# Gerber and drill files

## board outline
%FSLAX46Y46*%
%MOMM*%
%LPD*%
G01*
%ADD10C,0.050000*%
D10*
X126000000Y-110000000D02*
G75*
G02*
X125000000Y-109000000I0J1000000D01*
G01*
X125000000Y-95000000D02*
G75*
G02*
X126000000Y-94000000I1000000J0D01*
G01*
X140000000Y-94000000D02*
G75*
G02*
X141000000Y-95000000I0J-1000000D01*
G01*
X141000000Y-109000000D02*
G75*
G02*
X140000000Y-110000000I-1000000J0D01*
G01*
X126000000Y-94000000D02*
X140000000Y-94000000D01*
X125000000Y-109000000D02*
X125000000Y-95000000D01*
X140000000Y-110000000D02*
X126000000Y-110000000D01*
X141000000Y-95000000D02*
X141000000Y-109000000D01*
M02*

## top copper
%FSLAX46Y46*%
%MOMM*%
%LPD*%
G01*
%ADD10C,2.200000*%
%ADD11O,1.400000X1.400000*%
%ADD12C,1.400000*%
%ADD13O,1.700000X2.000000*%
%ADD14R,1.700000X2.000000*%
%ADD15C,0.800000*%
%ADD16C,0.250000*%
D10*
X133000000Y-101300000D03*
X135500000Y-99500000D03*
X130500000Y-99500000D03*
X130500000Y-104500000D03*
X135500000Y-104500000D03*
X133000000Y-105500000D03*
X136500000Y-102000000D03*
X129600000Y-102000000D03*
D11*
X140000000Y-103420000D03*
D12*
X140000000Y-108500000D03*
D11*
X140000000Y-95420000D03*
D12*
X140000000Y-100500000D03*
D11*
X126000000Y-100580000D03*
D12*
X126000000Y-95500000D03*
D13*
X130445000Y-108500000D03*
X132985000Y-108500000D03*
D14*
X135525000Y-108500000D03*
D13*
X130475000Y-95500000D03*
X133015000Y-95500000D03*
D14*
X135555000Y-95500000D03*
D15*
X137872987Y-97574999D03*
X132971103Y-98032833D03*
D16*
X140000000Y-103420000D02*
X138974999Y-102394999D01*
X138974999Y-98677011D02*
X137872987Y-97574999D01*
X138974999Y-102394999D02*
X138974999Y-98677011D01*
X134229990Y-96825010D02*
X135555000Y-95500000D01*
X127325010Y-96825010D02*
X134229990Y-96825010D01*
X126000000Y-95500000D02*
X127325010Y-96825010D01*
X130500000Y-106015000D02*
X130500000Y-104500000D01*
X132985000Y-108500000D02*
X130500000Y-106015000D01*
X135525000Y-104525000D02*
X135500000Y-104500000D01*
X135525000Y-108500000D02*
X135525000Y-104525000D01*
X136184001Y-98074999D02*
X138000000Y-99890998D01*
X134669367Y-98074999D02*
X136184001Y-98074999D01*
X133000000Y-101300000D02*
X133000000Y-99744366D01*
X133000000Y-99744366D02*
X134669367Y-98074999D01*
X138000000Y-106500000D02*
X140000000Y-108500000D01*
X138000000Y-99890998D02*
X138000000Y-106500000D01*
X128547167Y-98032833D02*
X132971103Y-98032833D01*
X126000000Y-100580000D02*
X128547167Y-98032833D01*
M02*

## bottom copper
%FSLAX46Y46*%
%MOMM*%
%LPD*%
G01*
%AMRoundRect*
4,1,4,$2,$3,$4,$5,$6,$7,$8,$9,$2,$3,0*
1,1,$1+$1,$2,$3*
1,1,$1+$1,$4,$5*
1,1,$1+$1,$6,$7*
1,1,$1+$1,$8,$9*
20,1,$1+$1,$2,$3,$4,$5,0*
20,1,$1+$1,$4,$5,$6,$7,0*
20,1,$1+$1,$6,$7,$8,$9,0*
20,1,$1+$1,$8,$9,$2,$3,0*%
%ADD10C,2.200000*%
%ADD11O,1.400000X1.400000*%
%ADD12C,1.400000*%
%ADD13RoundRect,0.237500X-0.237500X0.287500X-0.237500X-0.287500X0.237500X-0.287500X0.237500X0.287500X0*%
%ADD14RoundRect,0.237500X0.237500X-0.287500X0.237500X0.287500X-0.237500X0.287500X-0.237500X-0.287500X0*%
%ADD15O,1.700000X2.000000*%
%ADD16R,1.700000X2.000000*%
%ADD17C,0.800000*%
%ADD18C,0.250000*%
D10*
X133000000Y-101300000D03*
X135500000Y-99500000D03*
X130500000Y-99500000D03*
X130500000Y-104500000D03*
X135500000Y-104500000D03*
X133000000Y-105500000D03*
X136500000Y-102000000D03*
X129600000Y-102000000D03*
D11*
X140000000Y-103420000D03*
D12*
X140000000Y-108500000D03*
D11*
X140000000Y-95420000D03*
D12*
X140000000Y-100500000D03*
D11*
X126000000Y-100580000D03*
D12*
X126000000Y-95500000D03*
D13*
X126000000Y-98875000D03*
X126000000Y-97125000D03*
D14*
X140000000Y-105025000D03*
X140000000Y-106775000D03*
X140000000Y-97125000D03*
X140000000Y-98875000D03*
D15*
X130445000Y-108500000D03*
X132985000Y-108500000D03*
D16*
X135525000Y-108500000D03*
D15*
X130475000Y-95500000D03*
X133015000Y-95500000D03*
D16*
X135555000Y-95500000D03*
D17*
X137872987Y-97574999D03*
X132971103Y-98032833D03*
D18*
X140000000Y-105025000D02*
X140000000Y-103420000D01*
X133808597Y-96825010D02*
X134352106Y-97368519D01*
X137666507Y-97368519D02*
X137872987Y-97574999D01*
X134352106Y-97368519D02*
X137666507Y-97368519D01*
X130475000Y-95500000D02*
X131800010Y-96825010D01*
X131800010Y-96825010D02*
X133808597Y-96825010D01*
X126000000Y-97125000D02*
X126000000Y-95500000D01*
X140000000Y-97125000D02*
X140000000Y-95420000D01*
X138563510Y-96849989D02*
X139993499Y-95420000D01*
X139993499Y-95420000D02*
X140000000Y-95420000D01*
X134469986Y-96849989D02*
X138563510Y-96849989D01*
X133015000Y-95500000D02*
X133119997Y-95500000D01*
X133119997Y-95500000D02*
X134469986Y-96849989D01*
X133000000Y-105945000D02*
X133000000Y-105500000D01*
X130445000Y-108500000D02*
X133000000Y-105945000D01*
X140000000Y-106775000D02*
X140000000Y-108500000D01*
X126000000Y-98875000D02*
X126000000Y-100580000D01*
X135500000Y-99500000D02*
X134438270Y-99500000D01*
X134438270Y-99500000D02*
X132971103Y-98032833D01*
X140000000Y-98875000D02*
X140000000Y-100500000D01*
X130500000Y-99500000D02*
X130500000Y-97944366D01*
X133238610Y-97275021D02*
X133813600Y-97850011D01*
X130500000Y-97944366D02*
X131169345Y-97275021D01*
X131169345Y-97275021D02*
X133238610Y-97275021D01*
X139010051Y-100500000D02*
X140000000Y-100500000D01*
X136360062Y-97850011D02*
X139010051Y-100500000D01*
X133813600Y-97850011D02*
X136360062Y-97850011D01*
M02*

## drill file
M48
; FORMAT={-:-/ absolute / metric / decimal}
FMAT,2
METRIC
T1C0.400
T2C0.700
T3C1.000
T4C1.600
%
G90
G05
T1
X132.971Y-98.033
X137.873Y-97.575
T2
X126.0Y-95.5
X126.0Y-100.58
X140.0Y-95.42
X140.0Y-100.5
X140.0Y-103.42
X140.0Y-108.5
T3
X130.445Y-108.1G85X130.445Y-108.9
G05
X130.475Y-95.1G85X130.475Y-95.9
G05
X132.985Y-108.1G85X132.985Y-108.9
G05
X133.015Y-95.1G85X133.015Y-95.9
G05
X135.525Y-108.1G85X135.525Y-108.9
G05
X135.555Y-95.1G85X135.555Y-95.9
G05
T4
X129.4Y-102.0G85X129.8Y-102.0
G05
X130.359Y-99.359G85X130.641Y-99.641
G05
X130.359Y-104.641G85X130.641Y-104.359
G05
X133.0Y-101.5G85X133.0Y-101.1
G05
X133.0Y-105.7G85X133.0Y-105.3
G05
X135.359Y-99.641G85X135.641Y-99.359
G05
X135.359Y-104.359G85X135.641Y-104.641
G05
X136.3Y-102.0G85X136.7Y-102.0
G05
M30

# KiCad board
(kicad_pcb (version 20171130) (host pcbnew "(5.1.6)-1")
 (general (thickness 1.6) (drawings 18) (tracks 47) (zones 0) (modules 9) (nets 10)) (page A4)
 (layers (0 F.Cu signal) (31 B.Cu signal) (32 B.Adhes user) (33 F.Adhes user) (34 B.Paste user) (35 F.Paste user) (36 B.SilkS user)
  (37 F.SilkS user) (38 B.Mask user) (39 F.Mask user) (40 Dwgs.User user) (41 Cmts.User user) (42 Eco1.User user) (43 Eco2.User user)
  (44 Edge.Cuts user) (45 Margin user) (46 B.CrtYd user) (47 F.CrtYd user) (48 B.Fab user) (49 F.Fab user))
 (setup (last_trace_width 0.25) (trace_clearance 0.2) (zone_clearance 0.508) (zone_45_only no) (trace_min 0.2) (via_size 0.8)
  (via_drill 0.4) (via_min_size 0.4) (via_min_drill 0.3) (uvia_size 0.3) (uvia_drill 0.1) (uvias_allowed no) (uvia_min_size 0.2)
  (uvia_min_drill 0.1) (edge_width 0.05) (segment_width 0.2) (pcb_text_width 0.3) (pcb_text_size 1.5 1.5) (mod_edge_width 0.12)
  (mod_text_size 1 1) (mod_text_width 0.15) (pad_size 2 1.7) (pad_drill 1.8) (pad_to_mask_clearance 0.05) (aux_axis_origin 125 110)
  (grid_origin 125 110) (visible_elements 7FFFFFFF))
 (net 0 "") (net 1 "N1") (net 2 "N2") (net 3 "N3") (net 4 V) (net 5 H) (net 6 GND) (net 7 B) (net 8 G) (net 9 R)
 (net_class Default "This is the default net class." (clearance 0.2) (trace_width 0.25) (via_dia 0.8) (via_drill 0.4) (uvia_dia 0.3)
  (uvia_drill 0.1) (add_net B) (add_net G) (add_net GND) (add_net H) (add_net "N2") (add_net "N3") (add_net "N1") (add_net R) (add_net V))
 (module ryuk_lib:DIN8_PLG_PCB (layer B.Cu) (at 133 102 180)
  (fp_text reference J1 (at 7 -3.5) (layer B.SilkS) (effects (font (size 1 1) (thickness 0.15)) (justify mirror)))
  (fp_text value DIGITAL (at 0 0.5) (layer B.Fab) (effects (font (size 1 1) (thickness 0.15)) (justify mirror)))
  (pad 8 thru_hole circle (at 0 0.7 180) (size 2.2 2.2) (drill oval 1.6 2) (layers *.Cu *.Mask) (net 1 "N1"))
  (pad 6 thru_hole circle (at -2.5 2.5 135) (size 2.2 2.2) (drill oval 1.6 2) (layers *.Cu *.Mask) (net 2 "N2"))
  (pad 7 thru_hole circle (at 2.5 2.5 45) (size 2.2 2.2) (drill oval 1.6 2) (layers *.Cu *.Mask) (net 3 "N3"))
  (pad 5 thru_hole circle (at 2.5 -2.5 135) (size 2.2 2.2) (drill oval 1.6 2) (layers *.Cu *.Mask) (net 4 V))
  (pad 4 thru_hole circle (at -2.5 -2.5 45) (size 2.2 2.2) (drill oval 1.6 2) (layers *.Cu *.Mask) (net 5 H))
  (pad 2 thru_hole circle (at 0 -3.5 180) (size 2.2 2.2) (drill oval 1.6 2) (layers *.Cu *.Mask) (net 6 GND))
  (pad 1 thru_hole circle (at -3.5 0 90) (size 2.2 2.2) (drill oval 1.6 2) (layers *.Cu *.Mask))
  (pad 3 thru_hole circle (at 3.4 0 90) (size 2.2 2.2) (drill oval 1.6 2) (layers *.Cu *.Mask)))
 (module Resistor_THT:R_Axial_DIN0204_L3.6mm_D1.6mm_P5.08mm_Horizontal (layer F.Cu) (at 140 108.5 90)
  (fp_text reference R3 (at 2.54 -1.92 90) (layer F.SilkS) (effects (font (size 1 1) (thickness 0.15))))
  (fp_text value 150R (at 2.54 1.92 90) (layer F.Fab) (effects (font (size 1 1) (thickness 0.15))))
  (pad 2 thru_hole oval (at 5.08 0 90) (size 1.4 1.4) (drill 0.7) (layers *.Cu *.Mask) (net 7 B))
  (pad 1 thru_hole circle (at 0 0 90) (size 1.4 1.4) (drill 0.7) (layers *.Cu *.Mask) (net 1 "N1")))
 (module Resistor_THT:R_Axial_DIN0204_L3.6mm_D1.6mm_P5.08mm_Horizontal (layer F.Cu) (at 140 100.5 90)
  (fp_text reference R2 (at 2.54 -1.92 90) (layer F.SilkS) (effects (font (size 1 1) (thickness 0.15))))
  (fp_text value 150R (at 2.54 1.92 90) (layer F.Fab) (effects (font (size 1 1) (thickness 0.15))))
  (pad 2 thru_hole oval (at 5.08 0 90) (size 1.4 1.4) (drill 0.7) (layers *.Cu *.Mask) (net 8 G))
  (pad 1 thru_hole circle (at 0 0 90) (size 1.4 1.4) (drill 0.7) (layers *.Cu *.Mask) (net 3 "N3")))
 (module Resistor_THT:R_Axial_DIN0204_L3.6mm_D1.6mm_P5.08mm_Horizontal (layer F.Cu) (at 126 95.5 270)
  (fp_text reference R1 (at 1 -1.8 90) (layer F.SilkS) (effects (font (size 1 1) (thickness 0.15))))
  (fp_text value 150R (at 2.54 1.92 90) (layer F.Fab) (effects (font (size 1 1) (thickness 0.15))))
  (pad 2 thru_hole oval (at 5.08 0 270) (size 1.4 1.4) (drill 0.7) (layers *.Cu *.Mask) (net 2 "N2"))
  (pad 1 thru_hole circle (at 0 0 270) (size 1.4 1.4) (drill 0.7) (layers *.Cu *.Mask) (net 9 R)))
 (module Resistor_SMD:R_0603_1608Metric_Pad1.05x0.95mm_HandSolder (layer B.Cu) (at 126 98 270)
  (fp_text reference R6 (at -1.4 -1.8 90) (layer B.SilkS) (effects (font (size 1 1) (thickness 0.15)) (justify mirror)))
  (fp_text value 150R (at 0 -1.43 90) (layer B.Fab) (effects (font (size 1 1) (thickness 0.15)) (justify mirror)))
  (pad 2 smd roundrect (at 0.875 0 270) (size 1.05 0.95) (layers B.Cu B.Paste B.Mask) (roundrect_rratio 0.25) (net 2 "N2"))
  (pad 1 smd roundrect (at -0.875 0 270) (size 1.05 0.95) (layers B.Cu B.Paste B.Mask) (roundrect_rratio 0.25) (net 9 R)))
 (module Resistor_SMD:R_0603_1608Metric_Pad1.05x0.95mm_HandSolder (layer B.Cu) (at 140 105.9 90)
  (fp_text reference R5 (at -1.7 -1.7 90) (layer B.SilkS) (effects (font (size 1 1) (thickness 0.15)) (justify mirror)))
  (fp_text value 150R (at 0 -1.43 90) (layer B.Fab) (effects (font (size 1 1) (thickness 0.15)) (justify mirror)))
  (pad 2 smd roundrect (at 0.875 0 90) (size 1.05 0.95) (layers B.Cu B.Paste B.Mask) (roundrect_rratio 0.25) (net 7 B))
  (pad 1 smd roundrect (at -0.875 0 90) (size 1.05 0.95) (layers B.Cu B.Paste B.Mask) (roundrect_rratio 0.25) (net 1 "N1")))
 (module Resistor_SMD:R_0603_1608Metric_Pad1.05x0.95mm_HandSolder (layer B.Cu) (at 140 98 90)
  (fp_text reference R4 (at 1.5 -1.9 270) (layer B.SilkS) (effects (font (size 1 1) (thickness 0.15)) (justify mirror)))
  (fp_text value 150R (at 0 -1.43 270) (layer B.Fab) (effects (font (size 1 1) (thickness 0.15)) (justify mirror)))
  (pad 2 smd roundrect (at 0.875 0 90) (size 1.05 0.95) (layers B.Cu B.Paste B.Mask) (roundrect_rratio 0.25) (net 8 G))
  (pad 1 smd roundrect (at -0.875 0 90) (size 1.05 0.95) (layers B.Cu B.Paste B.Mask) (roundrect_rratio 0.25) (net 3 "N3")))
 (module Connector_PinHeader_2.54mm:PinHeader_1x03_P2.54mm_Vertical (layer F.Cu) (at 135.525 108.5 270)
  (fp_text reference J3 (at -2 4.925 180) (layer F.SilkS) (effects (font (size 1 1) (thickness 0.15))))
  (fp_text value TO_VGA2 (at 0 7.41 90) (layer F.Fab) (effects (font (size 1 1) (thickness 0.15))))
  (pad 3 thru_hole oval (at 0 5.08 270) (size 2 1.7) (drill oval 1.8 1) (layers *.Cu *.Mask) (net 6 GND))
  (pad 2 thru_hole oval (at 0 2.54 270) (size 2 1.7) (drill oval 1.8 1) (layers *.Cu *.Mask) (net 4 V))
  (pad 1 thru_hole rect (at 0 0 270) (size 2 1.7) (drill oval 1.8 1) (layers *.Cu *.Mask) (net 5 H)))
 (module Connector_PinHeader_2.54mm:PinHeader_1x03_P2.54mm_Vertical (layer F.Cu) (at 135.555 95.5 270)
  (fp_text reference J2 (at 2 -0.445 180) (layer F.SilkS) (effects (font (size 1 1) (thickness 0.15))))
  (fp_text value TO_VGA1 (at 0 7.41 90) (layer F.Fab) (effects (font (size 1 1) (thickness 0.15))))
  (pad 3 thru_hole oval (at 0 5.08 270) (size 2 1.7) (drill oval 1.8 1) (layers *.Cu *.Mask) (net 7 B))
  (pad 2 thru_hole oval (at 0 2.54 270) (size 2 1.7) (drill oval 1.8 1) (layers *.Cu *.Mask) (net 8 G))
  (pad 1 thru_hole rect (at 0 0 270) (size 2 1.7) (drill oval 1.8 1) (layers *.Cu *.Mask) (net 9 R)))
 (gr_arc (start 126 109) (end 125 109) (angle -90) (layer Edge.Cuts) (width 0.05))
 (gr_arc (start 126 95) (end 126 94) (angle -90) (layer Edge.Cuts) (width 0.05))
 (gr_arc (start 140 95) (end 141 95) (angle -90) (layer Edge.Cuts) (width 0.05))
 (gr_arc (start 140 109) (end 140 110) (angle -90) (layer Edge.Cuts) (width 0.05))
 (gr_line (start 126 94) (end 140 94) (layer Edge.Cuts) (width 0.05))
 (gr_line (start 125 109) (end 125 95) (layer Edge.Cuts) (width 0.05))
 (gr_line (start 140 110) (end 126 110) (layer Edge.Cuts) (width 0.05))
 (gr_line (start 141 95) (end 141 109) (layer Edge.Cuts) (width 0.05))
 (segment (start 140 105.025) (end 140 103.42) (width 0.25) (layer B.Cu) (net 7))
 (segment (start 140 103.42) (end 138.974999 102.394999) (width 0.25) (layer F.Cu) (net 7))
 (segment (start 133.808597 96.82501) (end 134.352106 97.368519) (width 0.25) (layer B.Cu) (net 7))
 (segment (start 138.974999 98.677011) (end 137.872987 97.574999) (width 0.25) (layer F.Cu) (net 7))
 (segment (start 137.666507 97.368519) (end 137.872987 97.574999) (width 0.25) (layer B.Cu) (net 7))
 (segment (start 134.352106 97.368519) (end 137.666507 97.368519) (width 0.25) (layer B.Cu) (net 7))
 (segment (start 130.475 95.5) (end 131.80001 96.82501) (width 0.25) (layer B.Cu) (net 7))
 (via (at 137.872987 97.574999) (size 0.8) (drill 0.4) (layers F.Cu B.Cu) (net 7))
 (segment (start 138.974999 102.394999) (end 138.974999 98.677011) (width 0.25) (layer F.Cu) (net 7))
 (segment (start 131.80001 96.82501) (end 133.808597 96.82501) (width 0.25) (layer B.Cu) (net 7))
 (segment (start 126 97.125) (end 126 95.5) (width 0.25) (layer B.Cu) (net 9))
 (segment (start 134.22999 96.82501) (end 135.555 95.5) (width 0.25) (layer F.Cu) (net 9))
 (segment (start 127.32501 96.82501) (end 134.22999 96.82501) (width 0.25) (layer F.Cu) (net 9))
 (segment (start 126 95.5) (end 127.32501 96.82501) (width 0.25) (layer F.Cu) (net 9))
 (segment (start 140 97.125) (end 140 95.42) (width 0.25) (layer B.Cu) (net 8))
 (segment (start 138.56351 96.849989) (end 139.993499 95.42) (width 0.25) (layer B.Cu) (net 8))
 (segment (start 139.993499 95.42) (end 140 95.42) (width 0.25) (layer B.Cu) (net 8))
 (segment (start 134.469986 96.849989) (end 138.56351 96.849989) (width 0.25) (layer B.Cu) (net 8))
 (segment (start 133.015 95.5) (end 133.119997 95.5) (width 0.25) (layer B.Cu) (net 8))
 (segment (start 133.119997 95.5) (end 134.469986 96.849989) (width 0.25) (layer B.Cu) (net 8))
 (segment (start 130.5 106.015) (end 130.5 104.5) (width 0.25) (layer F.Cu) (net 4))
 (segment (start 132.985 108.5) (end 130.5 106.015) (width 0.25) (layer F.Cu) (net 4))
 (segment (start 135.525 104.525) (end 135.5 104.5) (width 0.25) (layer F.Cu) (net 5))
 (segment (start 135.525 108.5) (end 135.525 104.525) (width 0.25) (layer F.Cu) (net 5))
 (segment (start 133 105.945) (end 133 105.5) (width 0.25) (layer B.Cu) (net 6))
 (segment (start 130.445 108.5) (end 133 105.945) (width 0.25) (layer B.Cu) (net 6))
 (segment (start 136.184001 98.074999) (end 138 99.890998) (width 0.25) (layer F.Cu) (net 1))
 (segment (start 134.669367 98.074999) (end 136.184001 98.074999) (width 0.25) (layer F.Cu) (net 1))
 (segment (start 133 101.3) (end 133 99.744366) (width 0.25) (layer F.Cu) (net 1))
 (segment (start 133 99.744366) (end 134.669367 98.074999) (width 0.25) (layer F.Cu) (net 1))
 (segment (start 138 106.5) (end 140 108.5) (width 0.25) (layer F.Cu) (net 1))
 (segment (start 138 99.890998) (end 138 106.5) (width 0.25) (layer F.Cu) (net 1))
 (segment (start 140 106.775) (end 140 108.5) (width 0.25) (layer B.Cu) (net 1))
 (segment (start 126 98.875) (end 126 100.58) (width 0.25) (layer B.Cu) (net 2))
 (segment (start 128.547167 98.032833) (end 132.971103 98.032833) (width 0.25) (layer F.Cu) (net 2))
 (via (at 132.971103 98.032833) (size 0.8) (drill 0.4) (layers F.Cu B.Cu) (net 2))
 (segment (start 135.5 99.5) (end 134.43827 99.5) (width 0.25) (layer B.Cu) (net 2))
 (segment (start 126 100.58) (end 128.547167 98.032833) (width 0.25) (layer F.Cu) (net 2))
 (segment (start 134.43827 99.5) (end 132.971103 98.032833) (width 0.25) (layer B.Cu) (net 2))
 (segment (start 140 98.875) (end 140 100.5) (width 0.25) (layer B.Cu) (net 3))
 (segment (start 130.5 99.5) (end 130.5 97.944366) (width 0.25) (layer B.Cu) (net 3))
 (segment (start 133.23861 97.275021) (end 133.8136 97.850011) (width 0.25) (layer B.Cu) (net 3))
 (segment (start 130.5 97.944366) (end 131.169345 97.275021) (width 0.25) (layer B.Cu) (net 3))
 (segment (start 131.169345 97.275021) (end 133.23861 97.275021) (width 0.25) (layer B.Cu) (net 3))
 (segment (start 139.010051 100.5) (end 140 100.5) (width 0.25) (layer B.Cu) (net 3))
 (segment (start 136.360062 97.850011) (end 139.010051 100.5) (width 0.25) (layer B.Cu) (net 3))
 (segment (start 133.8136 97.850011) (end 136.360062 97.850011) (width 0.25) (layer B.Cu) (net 3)))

